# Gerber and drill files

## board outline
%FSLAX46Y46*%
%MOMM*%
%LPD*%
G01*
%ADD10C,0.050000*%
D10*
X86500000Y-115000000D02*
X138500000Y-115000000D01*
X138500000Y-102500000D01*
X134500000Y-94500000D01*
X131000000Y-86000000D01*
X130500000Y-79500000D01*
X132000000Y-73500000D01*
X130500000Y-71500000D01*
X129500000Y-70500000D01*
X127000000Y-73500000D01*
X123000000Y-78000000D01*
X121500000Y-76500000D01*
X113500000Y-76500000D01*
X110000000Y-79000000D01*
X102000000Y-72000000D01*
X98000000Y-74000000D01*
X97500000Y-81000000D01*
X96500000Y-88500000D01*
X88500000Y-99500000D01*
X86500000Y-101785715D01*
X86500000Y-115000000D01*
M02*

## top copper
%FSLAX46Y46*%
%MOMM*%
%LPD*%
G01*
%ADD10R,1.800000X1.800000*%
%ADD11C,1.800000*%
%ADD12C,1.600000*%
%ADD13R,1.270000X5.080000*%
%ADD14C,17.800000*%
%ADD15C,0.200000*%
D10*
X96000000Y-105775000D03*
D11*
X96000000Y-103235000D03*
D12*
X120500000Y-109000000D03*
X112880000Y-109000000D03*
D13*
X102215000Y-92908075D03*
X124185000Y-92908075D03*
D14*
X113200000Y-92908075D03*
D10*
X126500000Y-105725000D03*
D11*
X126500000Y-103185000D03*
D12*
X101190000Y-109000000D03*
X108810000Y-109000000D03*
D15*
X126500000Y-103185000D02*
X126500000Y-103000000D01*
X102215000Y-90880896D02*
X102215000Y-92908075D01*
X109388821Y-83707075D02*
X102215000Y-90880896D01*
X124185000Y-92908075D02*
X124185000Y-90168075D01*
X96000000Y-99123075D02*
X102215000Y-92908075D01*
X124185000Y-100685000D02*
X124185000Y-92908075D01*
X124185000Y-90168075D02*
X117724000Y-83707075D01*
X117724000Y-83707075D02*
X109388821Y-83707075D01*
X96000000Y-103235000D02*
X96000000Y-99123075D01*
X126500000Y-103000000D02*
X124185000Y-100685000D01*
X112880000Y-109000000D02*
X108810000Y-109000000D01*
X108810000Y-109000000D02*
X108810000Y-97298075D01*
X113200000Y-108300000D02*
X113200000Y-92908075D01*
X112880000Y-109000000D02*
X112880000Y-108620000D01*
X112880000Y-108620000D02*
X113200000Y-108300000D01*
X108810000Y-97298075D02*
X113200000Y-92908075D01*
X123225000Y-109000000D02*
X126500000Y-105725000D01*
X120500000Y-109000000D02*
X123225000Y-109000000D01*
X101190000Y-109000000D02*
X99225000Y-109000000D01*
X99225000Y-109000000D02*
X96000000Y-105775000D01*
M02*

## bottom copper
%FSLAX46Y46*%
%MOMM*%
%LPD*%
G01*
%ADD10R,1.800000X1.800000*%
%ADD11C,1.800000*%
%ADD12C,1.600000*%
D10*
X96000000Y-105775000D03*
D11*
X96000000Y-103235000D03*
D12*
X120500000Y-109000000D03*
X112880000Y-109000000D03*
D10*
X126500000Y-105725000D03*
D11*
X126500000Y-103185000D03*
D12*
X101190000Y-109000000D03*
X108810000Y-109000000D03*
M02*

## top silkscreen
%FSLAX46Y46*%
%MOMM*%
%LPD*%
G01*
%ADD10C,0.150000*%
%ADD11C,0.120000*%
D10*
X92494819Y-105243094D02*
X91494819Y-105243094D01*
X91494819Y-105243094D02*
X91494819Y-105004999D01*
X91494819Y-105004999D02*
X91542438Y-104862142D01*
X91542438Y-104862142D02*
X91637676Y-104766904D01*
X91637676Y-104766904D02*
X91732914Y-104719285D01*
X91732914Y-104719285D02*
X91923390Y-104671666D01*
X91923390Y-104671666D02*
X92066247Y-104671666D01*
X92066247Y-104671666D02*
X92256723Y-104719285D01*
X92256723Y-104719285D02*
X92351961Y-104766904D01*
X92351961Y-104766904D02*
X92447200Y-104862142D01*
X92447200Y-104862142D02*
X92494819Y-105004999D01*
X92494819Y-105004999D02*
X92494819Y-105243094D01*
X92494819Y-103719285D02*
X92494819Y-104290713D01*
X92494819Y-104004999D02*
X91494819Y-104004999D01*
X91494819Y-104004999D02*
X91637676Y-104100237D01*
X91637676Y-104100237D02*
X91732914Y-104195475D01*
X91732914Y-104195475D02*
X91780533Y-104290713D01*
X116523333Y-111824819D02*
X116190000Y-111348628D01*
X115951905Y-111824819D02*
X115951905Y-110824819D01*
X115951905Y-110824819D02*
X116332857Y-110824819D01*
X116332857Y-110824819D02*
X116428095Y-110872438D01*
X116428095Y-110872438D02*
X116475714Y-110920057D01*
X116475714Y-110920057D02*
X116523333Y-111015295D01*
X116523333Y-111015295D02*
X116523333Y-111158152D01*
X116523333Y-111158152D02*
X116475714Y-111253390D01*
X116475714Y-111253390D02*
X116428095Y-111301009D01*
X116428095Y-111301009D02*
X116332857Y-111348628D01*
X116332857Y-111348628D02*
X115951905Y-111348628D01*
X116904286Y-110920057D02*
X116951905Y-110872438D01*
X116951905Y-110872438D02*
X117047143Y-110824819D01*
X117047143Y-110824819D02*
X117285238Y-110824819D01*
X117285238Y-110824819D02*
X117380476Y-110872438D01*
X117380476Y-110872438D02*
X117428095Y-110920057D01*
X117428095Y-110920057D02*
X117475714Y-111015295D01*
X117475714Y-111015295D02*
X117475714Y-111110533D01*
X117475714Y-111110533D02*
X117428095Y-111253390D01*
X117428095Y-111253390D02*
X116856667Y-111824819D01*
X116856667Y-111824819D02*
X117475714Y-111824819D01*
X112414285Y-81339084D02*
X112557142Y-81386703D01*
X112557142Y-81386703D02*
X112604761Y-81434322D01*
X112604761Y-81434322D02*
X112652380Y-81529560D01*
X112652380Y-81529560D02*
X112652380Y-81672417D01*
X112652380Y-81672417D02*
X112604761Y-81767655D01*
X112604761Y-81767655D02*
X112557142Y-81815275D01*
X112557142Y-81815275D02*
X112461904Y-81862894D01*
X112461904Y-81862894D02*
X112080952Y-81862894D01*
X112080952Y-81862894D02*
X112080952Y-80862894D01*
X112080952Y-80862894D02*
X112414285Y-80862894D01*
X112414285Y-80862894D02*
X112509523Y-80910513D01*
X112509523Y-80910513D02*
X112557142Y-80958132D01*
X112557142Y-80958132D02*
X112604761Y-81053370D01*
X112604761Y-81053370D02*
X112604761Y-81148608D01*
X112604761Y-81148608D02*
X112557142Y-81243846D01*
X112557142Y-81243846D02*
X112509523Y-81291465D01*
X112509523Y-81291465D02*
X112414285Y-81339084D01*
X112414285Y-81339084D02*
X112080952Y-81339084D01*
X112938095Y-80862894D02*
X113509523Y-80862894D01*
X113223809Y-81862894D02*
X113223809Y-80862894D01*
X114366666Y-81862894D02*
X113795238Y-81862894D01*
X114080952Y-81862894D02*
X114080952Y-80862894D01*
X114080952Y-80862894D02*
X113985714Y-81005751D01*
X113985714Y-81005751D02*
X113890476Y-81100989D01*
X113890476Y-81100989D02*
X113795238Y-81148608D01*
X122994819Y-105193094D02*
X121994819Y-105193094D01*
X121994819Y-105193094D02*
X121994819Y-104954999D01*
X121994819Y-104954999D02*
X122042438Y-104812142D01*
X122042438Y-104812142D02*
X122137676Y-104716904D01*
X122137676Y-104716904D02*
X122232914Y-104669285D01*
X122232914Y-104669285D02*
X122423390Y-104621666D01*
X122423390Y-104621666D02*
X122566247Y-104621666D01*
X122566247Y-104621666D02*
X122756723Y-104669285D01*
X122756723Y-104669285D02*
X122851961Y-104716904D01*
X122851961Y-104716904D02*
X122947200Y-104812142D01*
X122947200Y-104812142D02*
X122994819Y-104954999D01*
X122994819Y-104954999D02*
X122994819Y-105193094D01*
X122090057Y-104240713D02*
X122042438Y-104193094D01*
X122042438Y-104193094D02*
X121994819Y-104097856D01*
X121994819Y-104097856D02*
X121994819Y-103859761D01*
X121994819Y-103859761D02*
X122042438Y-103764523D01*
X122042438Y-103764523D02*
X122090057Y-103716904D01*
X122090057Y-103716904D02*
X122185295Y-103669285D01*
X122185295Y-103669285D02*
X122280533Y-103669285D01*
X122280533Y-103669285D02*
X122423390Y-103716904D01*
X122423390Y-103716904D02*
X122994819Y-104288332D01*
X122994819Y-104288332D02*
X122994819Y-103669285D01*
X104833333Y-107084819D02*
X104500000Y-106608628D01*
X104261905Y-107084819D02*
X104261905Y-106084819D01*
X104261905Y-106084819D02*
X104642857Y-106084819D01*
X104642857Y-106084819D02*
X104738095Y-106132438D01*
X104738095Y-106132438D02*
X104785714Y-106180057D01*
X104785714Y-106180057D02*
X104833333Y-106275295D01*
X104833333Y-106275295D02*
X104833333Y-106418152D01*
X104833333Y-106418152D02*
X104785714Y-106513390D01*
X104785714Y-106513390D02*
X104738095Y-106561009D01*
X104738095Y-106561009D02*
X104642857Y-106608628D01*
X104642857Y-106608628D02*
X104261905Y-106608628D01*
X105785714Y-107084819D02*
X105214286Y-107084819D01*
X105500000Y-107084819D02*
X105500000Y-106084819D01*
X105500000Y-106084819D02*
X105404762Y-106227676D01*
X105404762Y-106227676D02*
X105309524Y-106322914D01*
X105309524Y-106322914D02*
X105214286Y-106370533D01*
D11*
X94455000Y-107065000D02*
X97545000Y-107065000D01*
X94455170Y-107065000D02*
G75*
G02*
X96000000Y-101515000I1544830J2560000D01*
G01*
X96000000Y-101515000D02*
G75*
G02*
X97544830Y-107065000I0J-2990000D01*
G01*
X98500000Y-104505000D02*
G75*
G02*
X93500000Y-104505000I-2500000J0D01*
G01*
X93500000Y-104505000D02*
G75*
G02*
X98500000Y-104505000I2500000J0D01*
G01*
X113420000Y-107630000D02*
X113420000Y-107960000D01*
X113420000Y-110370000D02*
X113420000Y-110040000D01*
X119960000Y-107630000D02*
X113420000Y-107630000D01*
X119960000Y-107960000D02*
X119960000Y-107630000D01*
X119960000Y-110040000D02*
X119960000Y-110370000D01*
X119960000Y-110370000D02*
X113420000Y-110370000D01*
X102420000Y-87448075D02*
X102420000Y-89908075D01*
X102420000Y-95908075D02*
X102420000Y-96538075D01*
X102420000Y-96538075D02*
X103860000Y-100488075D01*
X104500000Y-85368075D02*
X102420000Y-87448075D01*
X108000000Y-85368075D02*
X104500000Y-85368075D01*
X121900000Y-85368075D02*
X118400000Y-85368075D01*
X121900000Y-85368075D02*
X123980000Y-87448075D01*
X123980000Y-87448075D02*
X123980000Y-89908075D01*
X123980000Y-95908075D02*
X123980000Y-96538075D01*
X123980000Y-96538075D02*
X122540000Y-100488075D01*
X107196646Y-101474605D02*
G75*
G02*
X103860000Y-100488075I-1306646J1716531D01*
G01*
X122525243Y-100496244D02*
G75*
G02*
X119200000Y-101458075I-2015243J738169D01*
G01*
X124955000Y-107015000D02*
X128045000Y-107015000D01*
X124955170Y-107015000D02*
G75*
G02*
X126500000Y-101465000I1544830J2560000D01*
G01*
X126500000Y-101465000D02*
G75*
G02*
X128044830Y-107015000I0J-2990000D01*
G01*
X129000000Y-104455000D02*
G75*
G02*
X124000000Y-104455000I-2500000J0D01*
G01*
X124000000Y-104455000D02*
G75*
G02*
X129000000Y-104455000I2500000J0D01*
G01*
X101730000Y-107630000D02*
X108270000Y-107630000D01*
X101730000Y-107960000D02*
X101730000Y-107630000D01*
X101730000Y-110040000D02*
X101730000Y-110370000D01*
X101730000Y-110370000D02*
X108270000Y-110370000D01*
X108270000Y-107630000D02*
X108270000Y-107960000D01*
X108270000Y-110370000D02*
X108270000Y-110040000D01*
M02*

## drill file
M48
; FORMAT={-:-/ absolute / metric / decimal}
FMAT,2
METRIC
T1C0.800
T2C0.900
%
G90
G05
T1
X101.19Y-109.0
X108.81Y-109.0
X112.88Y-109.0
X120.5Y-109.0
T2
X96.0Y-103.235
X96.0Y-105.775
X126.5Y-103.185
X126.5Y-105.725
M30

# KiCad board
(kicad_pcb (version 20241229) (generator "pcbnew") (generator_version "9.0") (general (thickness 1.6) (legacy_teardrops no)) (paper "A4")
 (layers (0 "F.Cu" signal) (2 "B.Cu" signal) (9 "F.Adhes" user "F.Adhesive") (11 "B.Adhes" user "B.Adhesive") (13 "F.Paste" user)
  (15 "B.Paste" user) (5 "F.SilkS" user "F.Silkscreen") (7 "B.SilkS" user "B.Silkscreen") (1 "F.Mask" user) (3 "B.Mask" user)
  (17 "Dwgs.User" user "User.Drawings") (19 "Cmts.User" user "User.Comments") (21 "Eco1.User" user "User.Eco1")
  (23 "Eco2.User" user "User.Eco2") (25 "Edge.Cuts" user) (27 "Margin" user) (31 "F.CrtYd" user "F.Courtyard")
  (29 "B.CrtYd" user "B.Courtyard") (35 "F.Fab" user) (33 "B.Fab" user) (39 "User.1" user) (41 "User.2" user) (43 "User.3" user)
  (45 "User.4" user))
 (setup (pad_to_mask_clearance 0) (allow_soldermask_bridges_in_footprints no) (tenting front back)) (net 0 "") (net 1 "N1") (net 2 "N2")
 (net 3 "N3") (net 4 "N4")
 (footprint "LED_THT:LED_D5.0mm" (layer "F.Cu") (at 96 105.775 90)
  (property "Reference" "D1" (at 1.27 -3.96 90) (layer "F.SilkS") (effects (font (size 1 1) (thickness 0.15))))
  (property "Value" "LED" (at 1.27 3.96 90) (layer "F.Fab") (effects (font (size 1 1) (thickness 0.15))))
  (fp_line (start -1.29 -1.545) (end -1.29 1.545) (stroke (width 0.12) (type solid)) (layer "F.SilkS"))
  (fp_arc (start -1.29 -1.54483) (mid 2.071779 -2.880495) (end 4.26 0) (stroke (width 0.12) (type solid)) (layer "F.SilkS"))
  (fp_arc (start 4.26 0) (mid 2.071779 2.880495) (end -1.29 1.54483) (stroke (width 0.12) (type solid)) (layer "F.SilkS"))
  (fp_circle (center 1.27 0) (end 3.77 0) (stroke (width 0.12) (type solid)) (fill no) (layer "F.SilkS"))
  (pad "1" thru_hole rect (at 0 0 90) (size 1.8 1.8) (drill 0.9) (layers "*.Cu" "*.Mask") (remove_unused_layers no) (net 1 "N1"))
  (pad "2" thru_hole circle (at 2.54 0 90) (size 1.8 1.8) (drill 0.9) (layers "*.Cu" "*.Mask") (remove_unused_layers no) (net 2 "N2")))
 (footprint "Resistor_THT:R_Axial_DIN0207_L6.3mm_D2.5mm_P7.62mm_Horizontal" (layer "F.Cu") (at 120.5 109 180)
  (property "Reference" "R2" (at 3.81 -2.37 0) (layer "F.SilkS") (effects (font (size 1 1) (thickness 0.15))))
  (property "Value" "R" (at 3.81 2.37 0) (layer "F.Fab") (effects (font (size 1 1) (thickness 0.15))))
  (fp_line (start 7.08 1.37) (end 7.08 1.04) (stroke (width 0.12) (type solid)) (layer "F.SilkS"))
  (fp_line (start 7.08 -1.37) (end 7.08 -1.04) (stroke (width 0.12) (type solid)) (layer "F.SilkS"))
  (fp_line (start 0.54 1.37) (end 7.08 1.37) (stroke (width 0.12) (type solid)) (layer "F.SilkS"))
  (fp_line (start 0.54 1.04) (end 0.54 1.37) (stroke (width 0.12) (type solid)) (layer "F.SilkS"))
  (fp_line (start 0.54 -1.04) (end 0.54 -1.37) (stroke (width 0.12) (type solid)) (layer "F.SilkS"))
  (fp_line (start 0.54 -1.37) (end 7.08 -1.37) (stroke (width 0.12) (type solid)) (layer "F.SilkS"))
  (pad "1" thru_hole circle (at 0 0 180) (size 1.6 1.6) (drill 0.8) (layers "*.Cu" "*.Mask") (remove_unused_layers no) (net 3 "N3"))
  (pad "2" thru_hole circle (at 7.62 0 180) (size 1.6 1.6) (drill 0.8) (layers "*.Cu" "*.Mask") (remove_unused_layers no) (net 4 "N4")))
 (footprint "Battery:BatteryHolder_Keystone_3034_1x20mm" (layer "F.Cu") (at 113.2 92.908075)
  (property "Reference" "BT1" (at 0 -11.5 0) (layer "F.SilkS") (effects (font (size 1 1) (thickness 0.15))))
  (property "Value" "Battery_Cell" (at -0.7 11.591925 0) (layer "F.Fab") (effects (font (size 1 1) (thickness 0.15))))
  (fp_line (start -10.78 -5.46) (end -10.78 -3) (stroke (width 0.12) (type solid)) (layer "F.SilkS"))
  (fp_line (start -10.78 3) (end -10.78 3.63) (stroke (width 0.12) (type solid)) (layer "F.SilkS"))
  (fp_line (start -10.78 3.63) (end -9.34 7.58) (stroke (width 0.12) (type solid)) (layer "F.SilkS"))
  (fp_line (start -8.7 -7.54) (end -10.78 -5.46) (stroke (width 0.12) (type solid)) (layer "F.SilkS"))
  (fp_line (start -5.2 -7.54) (end -8.7 -7.54) (stroke (width 0.12) (type solid)) (layer "F.SilkS"))
  (fp_line (start 8.7 -7.54) (end 5.2 -7.54) (stroke (width 0.12) (type solid)) (layer "F.SilkS"))
  (fp_line (start 8.7 -7.54) (end 10.78 -5.46) (stroke (width 0.12) (type solid)) (layer "F.SilkS"))
  (fp_line (start 10.78 -5.46) (end 10.78 -3) (stroke (width 0.12) (type solid)) (layer "F.SilkS"))
  (fp_line (start 10.78 3) (end 10.78 3.63) (stroke (width 0.12) (type solid)) (layer "F.SilkS"))
  (fp_line (start 10.78 3.63) (end 9.34 7.58) (stroke (width 0.12) (type solid)) (layer "F.SilkS"))
  (fp_arc (start -6.003354 8.56653) (mid -7.921654 8.918738) (end -9.34 7.58) (stroke (width 0.12) (type solid)) (layer "F.SilkS"))
  (fp_arc (start 9.325243 7.588169) (mid 7.90634 8.911668) (end 6 8.55) (stroke (width 0.12) (type solid)) (layer "F.SilkS"))
  (pad "1" smd rect (at -10.985 0) (size 1.27 5.08) (layers "F.Cu" "F.Mask" "F.Paste") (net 2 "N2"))
  (pad "1" smd rect (at 10.985 0) (size 1.27 5.08) (layers "F.Cu" "F.Mask" "F.Paste") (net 2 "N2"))
  (pad "2" smd circle (at 0 0) (size 17.8 17.8) (layers "F.Cu" "F.Mask") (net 4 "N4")))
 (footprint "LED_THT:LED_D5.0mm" (layer "F.Cu") (at 126.5 105.725 90)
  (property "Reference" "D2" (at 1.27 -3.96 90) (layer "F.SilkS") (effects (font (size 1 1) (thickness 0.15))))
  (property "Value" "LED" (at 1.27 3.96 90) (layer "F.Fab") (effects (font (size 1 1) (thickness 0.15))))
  (fp_line (start -1.29 -1.545) (end -1.29 1.545) (stroke (width 0.12) (type solid)) (layer "F.SilkS"))
  (fp_arc (start -1.29 -1.54483) (mid 2.071779 -2.880495) (end 4.26 0) (stroke (width 0.12) (type solid)) (layer "F.SilkS"))
  (fp_arc (start 4.26 0) (mid 2.071779 2.880495) (end -1.29 1.54483) (stroke (width 0.12) (type solid)) (layer "F.SilkS"))
  (fp_circle (center 1.27 0) (end 3.77 0) (stroke (width 0.12) (type solid)) (fill no) (layer "F.SilkS"))
  (pad "1" thru_hole rect (at 0 0 90) (size 1.8 1.8) (drill 0.9) (layers "*.Cu" "*.Mask") (remove_unused_layers no) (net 3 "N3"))
  (pad "2" thru_hole circle (at 2.54 0 90) (size 1.8 1.8) (drill 0.9) (layers "*.Cu" "*.Mask") (remove_unused_layers no) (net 2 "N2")))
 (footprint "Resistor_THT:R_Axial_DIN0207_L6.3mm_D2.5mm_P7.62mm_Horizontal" (layer "F.Cu") (at 101.19 109)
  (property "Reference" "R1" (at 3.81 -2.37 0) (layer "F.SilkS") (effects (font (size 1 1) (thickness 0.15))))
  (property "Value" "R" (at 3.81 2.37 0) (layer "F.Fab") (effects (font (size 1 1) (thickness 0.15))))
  (fp_line (start 0.54 -1.37) (end 7.08 -1.37) (stroke (width 0.12) (type solid)) (layer "F.SilkS"))
  (fp_line (start 0.54 -1.04) (end 0.54 -1.37) (stroke (width 0.12) (type solid)) (layer "F.SilkS"))
  (fp_line (start 0.54 1.04) (end 0.54 1.37) (stroke (width 0.12) (type solid)) (layer "F.SilkS"))
  (fp_line (start 0.54 1.37) (end 7.08 1.37) (stroke (width 0.12) (type solid)) (layer "F.SilkS"))
  (fp_line (start 7.08 -1.37) (end 7.08 -1.04) (stroke (width 0.12) (type solid)) (layer "F.SilkS"))
  (fp_line (start 7.08 1.37) (end 7.08 1.04) (stroke (width 0.12) (type solid)) (layer "F.SilkS"))
  (pad "1" thru_hole circle (at 0 0) (size 1.6 1.6) (drill 0.8) (layers "*.Cu" "*.Mask") (remove_unused_layers no) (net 1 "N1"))
  (pad "2" thru_hole circle (at 7.62 0) (size 1.6 1.6) (drill 0.8) (layers "*.Cu" "*.Mask") (remove_unused_layers no) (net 4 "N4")))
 (gr_poly
  (pts (xy 86.5 115) (xy 138.5 115) (xy 138.5 102.5) (xy 134.5 94.5) (xy 131 86) (xy 130.5 79.5) (xy 132 73.5) (xy 130.5 71.5)
   (xy 129.5 70.5) (xy 127 73.5) (xy 123 78) (xy 121.5 76.5) (xy 113.5 76.5) (xy 110 79) (xy 102 72) (xy 98 74) (xy 97.5 81) (xy 96.5 88.5)
   (xy 88.5 99.5) (xy 86.5 101.785715))
  (stroke (width 0.05) (type solid)) (fill no) (layer "Edge.Cuts"))
 (segment (start 126.5 103.185) (end 126.5 103) (width 0.2) (layer "F.Cu") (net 2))
 (segment (start 102.215 90.880896) (end 102.215 92.908075) (width 0.2) (layer "F.Cu") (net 2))
 (segment (start 109.388821 83.707075) (end 102.215 90.880896) (width 0.2) (layer "F.Cu") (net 2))
 (segment (start 124.185 92.908075) (end 124.185 90.168075) (width 0.2) (layer "F.Cu") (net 2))
 (segment (start 96 99.123075) (end 102.215 92.908075) (width 0.2) (layer "F.Cu") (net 2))
 (segment (start 124.185 100.685) (end 124.185 92.908075) (width 0.2) (layer "F.Cu") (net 2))
 (segment (start 124.185 90.168075) (end 117.724 83.707075) (width 0.2) (layer "F.Cu") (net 2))
 (segment (start 117.724 83.707075) (end 109.388821 83.707075) (width 0.2) (layer "F.Cu") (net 2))
 (segment (start 96 103.235) (end 96 99.123075) (width 0.2) (layer "F.Cu") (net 2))
 (segment (start 126.5 103) (end 124.185 100.685) (width 0.2) (layer "F.Cu") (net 2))
 (segment (start 112.88 109) (end 108.81 109) (width 0.2) (layer "F.Cu") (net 4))
 (segment (start 108.81 109) (end 108.81 97.298075) (width 0.2) (layer "F.Cu") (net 4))
 (segment (start 113.2 108.3) (end 113.2 92.908075) (width 0.2) (layer "F.Cu") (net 4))
 (segment (start 112.88 109) (end 112.88 108.62) (width 0.2) (layer "F.Cu") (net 4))
 (segment (start 112.88 108.62) (end 113.2 108.3) (width 0.2) (layer "F.Cu") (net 4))
 (segment (start 108.81 97.298075) (end 113.2 92.908075) (width 0.2) (layer "F.Cu") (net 4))
 (segment (start 123.225 109) (end 126.5 105.725) (width 0.2) (layer "F.Cu") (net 3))
 (segment (start 120.5 109) (end 123.225 109) (width 0.2) (layer "F.Cu") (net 3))
 (segment (start 101.19 109) (end 99.225 109) (width 0.2) (layer "F.Cu") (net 1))
 (segment (start 99.225 109) (end 96 105.775) (width 0.2) (layer "F.Cu") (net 1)))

